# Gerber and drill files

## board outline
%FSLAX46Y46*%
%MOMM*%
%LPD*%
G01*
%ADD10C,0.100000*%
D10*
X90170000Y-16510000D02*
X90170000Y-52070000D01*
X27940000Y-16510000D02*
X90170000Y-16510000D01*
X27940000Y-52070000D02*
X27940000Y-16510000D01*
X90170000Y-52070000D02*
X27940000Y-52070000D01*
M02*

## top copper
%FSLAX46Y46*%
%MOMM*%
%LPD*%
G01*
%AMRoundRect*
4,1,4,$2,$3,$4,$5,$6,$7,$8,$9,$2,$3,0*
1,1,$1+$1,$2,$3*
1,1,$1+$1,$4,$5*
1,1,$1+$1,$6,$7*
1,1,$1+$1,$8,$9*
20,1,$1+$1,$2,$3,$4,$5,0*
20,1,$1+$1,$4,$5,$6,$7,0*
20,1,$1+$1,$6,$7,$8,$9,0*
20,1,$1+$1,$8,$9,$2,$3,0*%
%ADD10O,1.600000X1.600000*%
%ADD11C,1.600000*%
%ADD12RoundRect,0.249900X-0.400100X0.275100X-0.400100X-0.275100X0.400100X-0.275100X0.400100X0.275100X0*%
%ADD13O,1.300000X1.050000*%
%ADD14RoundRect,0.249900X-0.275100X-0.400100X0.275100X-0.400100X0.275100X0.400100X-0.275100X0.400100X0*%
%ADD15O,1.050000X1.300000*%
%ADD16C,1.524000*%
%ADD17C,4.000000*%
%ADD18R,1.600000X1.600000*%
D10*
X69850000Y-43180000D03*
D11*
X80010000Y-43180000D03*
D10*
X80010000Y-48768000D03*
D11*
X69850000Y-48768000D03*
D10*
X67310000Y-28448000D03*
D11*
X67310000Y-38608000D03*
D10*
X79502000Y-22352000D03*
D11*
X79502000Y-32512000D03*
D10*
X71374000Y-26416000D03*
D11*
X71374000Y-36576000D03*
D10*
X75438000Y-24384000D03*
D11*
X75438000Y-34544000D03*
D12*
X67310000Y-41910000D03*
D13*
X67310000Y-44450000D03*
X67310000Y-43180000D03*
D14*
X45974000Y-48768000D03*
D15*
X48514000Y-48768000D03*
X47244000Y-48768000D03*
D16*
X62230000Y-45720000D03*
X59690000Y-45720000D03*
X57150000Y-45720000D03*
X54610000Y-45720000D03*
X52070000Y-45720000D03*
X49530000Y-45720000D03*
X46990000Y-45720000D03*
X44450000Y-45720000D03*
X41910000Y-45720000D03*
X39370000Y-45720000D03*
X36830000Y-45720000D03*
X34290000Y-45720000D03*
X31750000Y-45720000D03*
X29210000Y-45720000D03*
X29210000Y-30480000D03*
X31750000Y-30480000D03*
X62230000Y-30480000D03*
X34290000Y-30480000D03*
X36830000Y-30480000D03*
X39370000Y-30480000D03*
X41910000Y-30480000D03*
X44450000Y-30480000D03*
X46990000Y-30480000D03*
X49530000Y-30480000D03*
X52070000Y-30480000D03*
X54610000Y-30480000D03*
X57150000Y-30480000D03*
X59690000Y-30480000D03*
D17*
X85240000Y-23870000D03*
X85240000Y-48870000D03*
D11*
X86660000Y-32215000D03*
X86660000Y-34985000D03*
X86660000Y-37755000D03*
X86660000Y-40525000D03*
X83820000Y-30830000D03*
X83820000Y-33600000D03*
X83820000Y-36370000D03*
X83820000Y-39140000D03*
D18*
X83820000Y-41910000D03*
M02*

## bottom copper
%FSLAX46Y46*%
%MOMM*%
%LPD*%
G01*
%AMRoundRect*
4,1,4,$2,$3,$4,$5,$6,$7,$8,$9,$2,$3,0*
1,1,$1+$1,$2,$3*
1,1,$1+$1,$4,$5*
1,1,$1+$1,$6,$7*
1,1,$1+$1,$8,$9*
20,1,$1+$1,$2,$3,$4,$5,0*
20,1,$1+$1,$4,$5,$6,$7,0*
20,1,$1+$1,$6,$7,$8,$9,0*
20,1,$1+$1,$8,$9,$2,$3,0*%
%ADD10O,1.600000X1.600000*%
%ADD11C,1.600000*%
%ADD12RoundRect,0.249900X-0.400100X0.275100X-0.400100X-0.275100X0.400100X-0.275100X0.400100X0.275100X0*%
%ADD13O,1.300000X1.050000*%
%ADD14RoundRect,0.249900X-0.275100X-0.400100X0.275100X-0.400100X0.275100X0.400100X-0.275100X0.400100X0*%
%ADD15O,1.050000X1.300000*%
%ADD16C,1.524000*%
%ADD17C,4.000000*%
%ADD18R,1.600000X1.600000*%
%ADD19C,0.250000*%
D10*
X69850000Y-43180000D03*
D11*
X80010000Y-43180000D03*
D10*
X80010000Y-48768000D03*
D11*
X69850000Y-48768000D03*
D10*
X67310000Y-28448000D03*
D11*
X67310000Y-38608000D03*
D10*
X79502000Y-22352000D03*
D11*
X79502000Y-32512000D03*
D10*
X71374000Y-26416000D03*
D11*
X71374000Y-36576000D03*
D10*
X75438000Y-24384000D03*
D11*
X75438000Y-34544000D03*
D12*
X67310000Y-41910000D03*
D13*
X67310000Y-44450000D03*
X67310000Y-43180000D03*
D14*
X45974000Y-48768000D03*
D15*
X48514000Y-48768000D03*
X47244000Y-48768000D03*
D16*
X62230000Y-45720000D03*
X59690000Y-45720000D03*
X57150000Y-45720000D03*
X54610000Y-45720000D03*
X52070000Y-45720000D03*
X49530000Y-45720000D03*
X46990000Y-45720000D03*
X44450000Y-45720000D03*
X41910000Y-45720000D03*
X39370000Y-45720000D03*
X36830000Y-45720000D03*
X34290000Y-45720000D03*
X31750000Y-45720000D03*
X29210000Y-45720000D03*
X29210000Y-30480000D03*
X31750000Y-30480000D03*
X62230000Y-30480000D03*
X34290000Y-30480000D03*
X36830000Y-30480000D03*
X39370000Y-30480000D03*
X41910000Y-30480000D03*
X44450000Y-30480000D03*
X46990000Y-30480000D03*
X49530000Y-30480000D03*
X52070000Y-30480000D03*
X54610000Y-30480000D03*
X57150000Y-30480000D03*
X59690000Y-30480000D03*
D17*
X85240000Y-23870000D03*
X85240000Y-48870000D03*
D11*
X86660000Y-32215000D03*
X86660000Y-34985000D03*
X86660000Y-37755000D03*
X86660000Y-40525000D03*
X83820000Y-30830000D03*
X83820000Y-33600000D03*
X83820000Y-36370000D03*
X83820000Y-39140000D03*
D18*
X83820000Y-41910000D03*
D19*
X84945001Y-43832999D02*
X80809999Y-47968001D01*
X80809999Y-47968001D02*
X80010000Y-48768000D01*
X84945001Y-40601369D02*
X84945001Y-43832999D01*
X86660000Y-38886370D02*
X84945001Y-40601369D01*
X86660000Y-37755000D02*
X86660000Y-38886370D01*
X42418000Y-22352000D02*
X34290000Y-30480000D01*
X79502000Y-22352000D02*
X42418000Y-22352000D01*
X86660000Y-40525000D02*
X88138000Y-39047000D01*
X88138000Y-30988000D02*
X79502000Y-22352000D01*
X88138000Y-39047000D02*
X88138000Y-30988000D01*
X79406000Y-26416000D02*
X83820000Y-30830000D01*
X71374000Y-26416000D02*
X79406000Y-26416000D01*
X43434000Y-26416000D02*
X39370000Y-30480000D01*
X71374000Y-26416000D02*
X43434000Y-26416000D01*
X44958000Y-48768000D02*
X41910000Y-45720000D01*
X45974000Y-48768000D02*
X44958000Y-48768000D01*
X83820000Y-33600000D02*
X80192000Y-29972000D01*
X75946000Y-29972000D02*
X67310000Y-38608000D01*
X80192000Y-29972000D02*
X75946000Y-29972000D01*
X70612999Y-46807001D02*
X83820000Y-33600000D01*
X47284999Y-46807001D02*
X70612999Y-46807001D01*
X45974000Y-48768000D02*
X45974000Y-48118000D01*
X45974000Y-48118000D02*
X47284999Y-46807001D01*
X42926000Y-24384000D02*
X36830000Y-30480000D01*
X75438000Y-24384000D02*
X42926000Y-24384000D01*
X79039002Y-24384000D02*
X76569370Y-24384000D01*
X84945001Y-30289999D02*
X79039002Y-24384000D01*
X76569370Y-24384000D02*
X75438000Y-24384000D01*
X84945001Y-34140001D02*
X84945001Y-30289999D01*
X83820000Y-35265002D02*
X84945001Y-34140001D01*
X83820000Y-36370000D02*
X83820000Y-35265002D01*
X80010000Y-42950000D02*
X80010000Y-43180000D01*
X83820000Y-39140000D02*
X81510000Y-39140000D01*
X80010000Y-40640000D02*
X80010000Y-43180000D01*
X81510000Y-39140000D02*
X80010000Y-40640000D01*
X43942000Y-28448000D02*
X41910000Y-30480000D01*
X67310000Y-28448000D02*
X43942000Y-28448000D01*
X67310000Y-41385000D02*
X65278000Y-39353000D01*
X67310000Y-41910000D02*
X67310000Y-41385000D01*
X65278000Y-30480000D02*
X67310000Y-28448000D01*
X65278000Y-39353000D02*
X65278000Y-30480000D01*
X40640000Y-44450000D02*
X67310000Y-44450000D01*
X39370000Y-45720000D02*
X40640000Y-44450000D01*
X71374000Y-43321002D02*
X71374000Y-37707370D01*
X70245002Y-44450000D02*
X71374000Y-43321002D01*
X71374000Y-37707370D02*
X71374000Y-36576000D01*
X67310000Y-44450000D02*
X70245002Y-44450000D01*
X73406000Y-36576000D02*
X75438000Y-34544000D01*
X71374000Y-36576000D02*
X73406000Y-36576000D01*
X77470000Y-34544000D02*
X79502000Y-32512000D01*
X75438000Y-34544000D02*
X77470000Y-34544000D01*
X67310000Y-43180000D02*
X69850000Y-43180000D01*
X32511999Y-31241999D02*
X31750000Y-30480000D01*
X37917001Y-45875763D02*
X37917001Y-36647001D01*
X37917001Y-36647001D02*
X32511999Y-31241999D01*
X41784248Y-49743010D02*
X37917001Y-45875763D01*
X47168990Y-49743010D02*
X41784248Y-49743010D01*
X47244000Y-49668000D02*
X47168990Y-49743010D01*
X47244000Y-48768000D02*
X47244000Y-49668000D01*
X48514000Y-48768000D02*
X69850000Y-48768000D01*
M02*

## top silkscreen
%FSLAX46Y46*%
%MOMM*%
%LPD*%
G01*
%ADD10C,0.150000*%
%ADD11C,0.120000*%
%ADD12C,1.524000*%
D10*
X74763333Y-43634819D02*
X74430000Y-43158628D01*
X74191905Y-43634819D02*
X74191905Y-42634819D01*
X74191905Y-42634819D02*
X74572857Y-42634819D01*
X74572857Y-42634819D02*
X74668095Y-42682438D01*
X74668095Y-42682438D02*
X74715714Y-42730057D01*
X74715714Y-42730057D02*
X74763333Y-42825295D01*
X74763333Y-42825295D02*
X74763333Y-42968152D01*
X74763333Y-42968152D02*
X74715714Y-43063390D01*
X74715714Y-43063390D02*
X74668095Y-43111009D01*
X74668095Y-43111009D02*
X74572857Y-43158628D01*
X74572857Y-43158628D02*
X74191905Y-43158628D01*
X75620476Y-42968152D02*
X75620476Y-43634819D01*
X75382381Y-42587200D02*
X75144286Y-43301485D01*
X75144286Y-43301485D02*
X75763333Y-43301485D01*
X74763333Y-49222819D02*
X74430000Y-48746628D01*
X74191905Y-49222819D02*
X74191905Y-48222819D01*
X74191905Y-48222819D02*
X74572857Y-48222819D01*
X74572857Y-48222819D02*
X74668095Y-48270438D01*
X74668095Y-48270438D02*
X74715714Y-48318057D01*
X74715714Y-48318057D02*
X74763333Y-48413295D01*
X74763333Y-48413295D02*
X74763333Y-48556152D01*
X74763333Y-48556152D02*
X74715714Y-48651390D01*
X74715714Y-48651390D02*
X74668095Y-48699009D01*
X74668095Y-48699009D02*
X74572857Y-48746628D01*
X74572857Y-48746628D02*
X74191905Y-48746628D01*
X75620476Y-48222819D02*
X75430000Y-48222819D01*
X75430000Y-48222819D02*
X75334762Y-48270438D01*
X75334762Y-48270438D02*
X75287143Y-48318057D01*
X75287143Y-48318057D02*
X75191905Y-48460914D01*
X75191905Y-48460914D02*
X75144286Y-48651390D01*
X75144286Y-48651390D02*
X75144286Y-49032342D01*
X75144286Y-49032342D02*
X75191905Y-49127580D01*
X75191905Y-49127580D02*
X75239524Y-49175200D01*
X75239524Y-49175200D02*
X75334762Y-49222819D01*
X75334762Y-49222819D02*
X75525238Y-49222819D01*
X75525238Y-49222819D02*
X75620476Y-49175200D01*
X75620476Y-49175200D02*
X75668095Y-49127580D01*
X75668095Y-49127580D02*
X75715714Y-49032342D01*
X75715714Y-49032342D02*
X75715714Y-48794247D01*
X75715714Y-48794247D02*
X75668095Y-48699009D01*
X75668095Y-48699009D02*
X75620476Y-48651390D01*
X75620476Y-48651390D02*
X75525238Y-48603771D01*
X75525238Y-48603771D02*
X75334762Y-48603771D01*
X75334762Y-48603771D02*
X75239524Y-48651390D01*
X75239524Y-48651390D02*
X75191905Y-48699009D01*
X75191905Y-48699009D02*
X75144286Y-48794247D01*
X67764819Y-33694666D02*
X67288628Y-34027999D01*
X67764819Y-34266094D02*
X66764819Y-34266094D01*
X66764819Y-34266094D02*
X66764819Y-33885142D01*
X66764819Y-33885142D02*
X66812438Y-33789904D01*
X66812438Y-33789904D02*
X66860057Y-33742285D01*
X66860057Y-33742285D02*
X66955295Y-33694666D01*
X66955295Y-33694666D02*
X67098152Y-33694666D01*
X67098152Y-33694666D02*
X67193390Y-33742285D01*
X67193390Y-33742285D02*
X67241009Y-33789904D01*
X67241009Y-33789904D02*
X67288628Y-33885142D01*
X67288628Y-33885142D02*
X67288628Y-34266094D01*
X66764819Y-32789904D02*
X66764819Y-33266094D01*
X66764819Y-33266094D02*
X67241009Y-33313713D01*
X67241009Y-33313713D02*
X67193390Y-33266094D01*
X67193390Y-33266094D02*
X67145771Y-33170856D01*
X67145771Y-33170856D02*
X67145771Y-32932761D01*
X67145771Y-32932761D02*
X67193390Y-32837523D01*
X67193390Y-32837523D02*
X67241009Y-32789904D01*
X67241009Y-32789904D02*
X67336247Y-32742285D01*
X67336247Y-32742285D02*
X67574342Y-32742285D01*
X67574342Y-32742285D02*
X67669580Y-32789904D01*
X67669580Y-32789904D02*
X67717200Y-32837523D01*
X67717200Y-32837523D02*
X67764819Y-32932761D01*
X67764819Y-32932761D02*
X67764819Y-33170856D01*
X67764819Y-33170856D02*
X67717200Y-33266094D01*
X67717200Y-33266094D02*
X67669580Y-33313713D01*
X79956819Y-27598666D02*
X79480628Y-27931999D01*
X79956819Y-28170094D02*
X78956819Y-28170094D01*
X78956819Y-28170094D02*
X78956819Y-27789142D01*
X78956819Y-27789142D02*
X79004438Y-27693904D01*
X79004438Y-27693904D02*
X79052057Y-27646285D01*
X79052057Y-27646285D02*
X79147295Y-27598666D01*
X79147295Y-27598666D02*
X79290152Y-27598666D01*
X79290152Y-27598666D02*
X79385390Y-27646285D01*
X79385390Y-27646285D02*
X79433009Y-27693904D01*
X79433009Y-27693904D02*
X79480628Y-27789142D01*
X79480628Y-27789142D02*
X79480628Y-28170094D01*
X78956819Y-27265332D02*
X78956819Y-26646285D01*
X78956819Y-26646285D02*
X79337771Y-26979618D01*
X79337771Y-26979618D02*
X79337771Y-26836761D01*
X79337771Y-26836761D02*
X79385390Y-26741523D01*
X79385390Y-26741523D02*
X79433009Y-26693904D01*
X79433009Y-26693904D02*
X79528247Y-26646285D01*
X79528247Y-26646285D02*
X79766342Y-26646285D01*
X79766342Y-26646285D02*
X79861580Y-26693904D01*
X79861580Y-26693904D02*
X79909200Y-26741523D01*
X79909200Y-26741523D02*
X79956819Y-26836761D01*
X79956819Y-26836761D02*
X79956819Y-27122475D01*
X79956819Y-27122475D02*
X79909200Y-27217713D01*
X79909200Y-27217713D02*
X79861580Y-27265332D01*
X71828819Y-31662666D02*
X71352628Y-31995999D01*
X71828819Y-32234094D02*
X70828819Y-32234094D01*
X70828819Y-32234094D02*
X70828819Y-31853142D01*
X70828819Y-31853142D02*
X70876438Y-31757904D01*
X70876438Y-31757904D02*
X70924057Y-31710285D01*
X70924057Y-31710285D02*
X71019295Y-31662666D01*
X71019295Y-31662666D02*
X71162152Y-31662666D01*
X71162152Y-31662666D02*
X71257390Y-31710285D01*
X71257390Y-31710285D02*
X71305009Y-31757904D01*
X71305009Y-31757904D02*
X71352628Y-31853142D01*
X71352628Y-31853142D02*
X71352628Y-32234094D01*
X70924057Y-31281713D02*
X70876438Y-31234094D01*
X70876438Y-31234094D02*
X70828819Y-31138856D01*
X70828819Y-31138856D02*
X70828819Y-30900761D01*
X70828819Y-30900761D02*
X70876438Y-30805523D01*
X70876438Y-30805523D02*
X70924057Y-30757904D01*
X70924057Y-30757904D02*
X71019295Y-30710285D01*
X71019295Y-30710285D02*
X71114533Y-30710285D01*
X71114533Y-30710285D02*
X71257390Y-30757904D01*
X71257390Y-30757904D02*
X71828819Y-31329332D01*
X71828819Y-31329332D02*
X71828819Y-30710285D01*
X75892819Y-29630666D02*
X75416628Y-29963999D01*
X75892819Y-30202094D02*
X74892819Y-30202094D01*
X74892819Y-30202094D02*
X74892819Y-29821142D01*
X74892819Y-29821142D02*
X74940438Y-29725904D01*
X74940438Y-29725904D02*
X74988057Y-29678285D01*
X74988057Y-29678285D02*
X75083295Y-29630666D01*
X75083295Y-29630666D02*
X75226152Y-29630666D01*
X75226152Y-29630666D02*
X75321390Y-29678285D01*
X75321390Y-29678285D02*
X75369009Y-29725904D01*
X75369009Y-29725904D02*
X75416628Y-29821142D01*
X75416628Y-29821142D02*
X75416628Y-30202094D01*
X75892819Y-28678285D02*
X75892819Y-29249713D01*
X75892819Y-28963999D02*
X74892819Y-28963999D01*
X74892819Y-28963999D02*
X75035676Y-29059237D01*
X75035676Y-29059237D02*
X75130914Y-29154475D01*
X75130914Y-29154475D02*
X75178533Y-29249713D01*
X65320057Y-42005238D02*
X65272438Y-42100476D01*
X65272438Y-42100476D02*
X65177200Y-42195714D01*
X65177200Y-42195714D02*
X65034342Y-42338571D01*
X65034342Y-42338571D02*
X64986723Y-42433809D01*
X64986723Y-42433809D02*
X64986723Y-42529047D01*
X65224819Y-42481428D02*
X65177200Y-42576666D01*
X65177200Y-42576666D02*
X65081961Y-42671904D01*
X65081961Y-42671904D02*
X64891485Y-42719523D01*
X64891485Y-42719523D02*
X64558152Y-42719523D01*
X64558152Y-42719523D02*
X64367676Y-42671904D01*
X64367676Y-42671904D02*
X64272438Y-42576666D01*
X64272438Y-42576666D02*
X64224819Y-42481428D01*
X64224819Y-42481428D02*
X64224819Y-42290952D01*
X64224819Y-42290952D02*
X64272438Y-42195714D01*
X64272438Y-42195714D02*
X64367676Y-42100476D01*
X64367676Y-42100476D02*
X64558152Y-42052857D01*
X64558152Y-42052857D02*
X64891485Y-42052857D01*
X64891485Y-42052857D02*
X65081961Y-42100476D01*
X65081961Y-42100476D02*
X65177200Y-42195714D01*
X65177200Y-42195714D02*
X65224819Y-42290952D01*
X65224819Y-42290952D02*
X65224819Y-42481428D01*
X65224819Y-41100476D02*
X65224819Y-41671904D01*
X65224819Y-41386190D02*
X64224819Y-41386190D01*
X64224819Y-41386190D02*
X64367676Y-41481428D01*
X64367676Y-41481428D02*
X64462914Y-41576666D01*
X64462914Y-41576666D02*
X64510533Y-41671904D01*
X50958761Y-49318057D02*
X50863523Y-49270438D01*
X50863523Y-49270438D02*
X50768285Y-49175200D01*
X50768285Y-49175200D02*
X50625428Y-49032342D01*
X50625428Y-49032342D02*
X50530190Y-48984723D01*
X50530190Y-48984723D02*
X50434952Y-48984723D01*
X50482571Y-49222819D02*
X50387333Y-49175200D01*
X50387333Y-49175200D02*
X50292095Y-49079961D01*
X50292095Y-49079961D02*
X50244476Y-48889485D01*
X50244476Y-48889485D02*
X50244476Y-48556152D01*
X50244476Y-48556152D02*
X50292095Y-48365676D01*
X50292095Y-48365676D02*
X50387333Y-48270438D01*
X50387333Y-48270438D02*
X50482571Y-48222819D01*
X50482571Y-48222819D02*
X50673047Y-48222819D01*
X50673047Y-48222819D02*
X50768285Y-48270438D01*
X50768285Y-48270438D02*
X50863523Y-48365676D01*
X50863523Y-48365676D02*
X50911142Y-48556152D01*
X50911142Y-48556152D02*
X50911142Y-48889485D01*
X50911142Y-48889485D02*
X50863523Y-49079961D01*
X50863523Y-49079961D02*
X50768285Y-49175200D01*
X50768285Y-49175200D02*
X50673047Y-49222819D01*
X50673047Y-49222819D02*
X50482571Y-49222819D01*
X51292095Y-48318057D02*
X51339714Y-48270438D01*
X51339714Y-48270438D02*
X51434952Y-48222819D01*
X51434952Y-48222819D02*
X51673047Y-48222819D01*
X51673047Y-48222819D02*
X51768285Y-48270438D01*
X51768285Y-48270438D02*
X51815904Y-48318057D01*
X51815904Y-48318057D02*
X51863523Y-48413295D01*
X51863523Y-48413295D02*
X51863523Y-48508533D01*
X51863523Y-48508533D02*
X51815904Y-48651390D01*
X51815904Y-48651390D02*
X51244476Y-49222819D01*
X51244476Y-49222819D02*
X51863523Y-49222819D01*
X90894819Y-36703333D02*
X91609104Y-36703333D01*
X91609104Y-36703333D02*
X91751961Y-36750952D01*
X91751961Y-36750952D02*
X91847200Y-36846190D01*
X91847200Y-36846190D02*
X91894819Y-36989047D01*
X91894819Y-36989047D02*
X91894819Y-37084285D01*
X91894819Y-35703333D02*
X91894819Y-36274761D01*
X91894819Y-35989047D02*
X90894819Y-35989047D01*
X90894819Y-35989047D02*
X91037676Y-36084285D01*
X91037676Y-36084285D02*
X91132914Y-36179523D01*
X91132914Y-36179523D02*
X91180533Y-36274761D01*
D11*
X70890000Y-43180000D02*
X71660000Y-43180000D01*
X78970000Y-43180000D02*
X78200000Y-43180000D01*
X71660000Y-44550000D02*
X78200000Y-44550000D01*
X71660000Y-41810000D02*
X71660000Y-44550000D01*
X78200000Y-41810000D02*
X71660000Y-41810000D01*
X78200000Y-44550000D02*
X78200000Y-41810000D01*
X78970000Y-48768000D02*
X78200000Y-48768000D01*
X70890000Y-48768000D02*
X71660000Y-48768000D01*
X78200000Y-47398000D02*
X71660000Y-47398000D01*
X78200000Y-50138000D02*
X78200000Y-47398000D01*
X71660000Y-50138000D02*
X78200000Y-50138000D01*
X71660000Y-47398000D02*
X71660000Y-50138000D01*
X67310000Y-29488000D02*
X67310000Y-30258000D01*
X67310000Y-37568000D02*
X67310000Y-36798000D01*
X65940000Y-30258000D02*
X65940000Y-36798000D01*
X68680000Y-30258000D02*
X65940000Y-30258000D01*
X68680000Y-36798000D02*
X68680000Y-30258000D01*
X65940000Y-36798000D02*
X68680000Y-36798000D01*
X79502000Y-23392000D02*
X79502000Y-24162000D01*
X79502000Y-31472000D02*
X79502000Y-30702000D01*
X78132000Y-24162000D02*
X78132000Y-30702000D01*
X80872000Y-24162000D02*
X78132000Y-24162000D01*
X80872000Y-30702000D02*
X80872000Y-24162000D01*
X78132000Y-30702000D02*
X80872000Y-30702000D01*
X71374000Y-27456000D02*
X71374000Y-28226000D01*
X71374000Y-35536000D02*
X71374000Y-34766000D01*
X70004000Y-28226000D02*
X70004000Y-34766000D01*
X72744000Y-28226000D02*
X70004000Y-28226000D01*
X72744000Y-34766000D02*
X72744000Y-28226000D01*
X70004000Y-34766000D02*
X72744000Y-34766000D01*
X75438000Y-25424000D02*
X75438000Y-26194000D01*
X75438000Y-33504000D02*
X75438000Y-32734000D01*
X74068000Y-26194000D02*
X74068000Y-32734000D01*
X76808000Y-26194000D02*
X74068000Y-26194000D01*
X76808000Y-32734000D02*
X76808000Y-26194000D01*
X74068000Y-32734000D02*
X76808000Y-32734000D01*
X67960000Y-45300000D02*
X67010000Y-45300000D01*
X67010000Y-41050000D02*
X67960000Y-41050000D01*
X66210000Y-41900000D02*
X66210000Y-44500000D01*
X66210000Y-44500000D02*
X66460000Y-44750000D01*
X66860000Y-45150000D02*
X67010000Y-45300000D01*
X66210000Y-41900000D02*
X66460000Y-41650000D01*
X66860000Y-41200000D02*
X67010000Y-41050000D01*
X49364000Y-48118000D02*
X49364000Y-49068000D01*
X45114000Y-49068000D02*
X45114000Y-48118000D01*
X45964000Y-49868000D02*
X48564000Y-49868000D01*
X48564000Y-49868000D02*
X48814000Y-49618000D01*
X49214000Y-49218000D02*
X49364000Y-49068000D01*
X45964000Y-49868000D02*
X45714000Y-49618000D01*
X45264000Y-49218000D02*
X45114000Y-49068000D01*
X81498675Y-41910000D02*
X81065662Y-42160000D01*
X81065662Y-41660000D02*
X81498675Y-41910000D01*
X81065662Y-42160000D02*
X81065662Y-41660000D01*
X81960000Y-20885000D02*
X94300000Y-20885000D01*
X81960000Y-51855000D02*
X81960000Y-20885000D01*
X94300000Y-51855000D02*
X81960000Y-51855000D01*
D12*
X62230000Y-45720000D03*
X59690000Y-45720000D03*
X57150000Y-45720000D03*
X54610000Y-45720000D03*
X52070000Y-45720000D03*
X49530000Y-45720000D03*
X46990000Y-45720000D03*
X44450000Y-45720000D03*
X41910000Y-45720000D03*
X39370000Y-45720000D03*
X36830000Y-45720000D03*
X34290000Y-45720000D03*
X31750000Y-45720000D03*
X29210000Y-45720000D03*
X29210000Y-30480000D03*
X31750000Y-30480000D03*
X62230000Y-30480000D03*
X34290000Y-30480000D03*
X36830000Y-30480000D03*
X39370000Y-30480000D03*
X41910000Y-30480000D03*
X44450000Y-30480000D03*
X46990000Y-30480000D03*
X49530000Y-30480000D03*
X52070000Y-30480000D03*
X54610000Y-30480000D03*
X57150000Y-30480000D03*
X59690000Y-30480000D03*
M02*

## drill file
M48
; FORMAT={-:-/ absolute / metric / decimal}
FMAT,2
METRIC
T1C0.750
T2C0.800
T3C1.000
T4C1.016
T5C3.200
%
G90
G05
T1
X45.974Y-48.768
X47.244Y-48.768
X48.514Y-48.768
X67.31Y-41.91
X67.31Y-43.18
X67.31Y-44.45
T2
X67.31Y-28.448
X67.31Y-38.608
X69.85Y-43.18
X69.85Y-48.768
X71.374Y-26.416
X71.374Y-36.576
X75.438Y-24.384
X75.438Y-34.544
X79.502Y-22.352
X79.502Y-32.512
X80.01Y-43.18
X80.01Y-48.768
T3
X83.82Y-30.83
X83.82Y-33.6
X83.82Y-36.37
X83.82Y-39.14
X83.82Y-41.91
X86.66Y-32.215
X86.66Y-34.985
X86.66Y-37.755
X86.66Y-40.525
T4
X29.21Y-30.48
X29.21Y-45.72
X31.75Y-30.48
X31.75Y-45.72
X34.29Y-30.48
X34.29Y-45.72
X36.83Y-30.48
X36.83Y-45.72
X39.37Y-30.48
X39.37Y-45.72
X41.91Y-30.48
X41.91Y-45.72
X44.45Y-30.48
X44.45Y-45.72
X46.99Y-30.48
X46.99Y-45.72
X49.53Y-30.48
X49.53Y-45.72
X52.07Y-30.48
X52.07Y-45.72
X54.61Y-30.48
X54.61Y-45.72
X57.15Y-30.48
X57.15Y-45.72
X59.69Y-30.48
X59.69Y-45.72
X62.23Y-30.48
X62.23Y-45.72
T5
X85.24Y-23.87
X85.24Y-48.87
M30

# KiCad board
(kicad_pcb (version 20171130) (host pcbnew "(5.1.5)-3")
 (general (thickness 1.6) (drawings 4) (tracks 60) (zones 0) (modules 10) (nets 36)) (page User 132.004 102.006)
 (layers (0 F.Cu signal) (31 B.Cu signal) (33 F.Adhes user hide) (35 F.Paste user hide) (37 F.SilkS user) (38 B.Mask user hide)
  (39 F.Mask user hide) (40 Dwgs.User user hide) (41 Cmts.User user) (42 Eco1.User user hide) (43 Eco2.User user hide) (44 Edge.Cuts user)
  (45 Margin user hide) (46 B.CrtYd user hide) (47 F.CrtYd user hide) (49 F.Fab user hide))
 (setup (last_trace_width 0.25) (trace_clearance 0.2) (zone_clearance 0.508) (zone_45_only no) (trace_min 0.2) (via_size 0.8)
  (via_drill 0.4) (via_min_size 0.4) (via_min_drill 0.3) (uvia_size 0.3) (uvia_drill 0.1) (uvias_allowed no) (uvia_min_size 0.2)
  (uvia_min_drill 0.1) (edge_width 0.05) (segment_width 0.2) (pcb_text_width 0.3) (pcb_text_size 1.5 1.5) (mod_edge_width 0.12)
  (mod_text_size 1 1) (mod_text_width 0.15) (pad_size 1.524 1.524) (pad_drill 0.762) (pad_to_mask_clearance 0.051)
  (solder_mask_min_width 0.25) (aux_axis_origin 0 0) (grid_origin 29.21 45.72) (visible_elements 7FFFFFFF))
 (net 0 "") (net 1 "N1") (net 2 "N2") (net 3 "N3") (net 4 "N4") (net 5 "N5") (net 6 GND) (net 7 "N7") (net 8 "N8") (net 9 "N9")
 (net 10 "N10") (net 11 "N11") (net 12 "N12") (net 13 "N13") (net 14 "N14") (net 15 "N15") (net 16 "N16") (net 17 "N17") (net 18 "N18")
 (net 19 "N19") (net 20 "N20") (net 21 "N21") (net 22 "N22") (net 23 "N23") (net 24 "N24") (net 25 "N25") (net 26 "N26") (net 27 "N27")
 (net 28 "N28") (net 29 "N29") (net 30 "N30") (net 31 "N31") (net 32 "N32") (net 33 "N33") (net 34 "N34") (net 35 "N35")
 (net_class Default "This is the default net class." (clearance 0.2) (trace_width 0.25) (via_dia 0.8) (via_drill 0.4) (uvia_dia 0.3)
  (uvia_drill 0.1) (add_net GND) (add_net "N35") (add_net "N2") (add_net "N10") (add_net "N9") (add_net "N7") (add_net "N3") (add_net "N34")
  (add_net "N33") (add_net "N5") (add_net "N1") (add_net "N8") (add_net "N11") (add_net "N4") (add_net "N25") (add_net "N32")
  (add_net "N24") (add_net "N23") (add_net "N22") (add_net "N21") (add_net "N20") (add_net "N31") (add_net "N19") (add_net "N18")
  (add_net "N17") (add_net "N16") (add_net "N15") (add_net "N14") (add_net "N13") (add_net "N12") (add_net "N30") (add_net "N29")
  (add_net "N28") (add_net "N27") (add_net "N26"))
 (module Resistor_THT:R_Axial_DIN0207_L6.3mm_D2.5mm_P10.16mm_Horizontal (layer F.Cu) (at 80.01 43.18 180)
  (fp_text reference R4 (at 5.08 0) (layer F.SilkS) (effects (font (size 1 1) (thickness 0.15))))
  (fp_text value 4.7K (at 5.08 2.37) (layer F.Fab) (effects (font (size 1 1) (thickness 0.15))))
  (fp_line (start 9.12 0) (end 8.35 0) (layer F.SilkS) (width 0.12))
  (fp_line (start 1.04 0) (end 1.81 0) (layer F.SilkS) (width 0.12))
  (fp_line (start 8.35 -1.37) (end 1.81 -1.37) (layer F.SilkS) (width 0.12))
  (fp_line (start 8.35 1.37) (end 8.35 -1.37) (layer F.SilkS) (width 0.12))
  (fp_line (start 1.81 1.37) (end 8.35 1.37) (layer F.SilkS) (width 0.12))
  (fp_line (start 1.81 -1.37) (end 1.81 1.37) (layer F.SilkS) (width 0.12))
  (pad 2 thru_hole oval (at 10.16 0 180) (size 1.6 1.6) (drill 0.8) (layers *.Cu *.Mask) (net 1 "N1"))
  (pad 1 thru_hole circle (at 0 0 180) (size 1.6 1.6) (drill 0.8) (layers *.Cu *.Mask) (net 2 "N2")))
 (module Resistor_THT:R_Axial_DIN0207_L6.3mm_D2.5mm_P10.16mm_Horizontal (layer F.Cu) (at 69.85 48.768)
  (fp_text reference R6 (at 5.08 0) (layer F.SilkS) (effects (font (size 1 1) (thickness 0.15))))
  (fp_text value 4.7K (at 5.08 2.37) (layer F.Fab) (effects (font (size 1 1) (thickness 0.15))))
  (fp_line (start 9.12 0) (end 8.35 0) (layer F.SilkS) (width 0.12))
  (fp_line (start 1.04 0) (end 1.81 0) (layer F.SilkS) (width 0.12))
  (fp_line (start 8.35 -1.37) (end 1.81 -1.37) (layer F.SilkS) (width 0.12))
  (fp_line (start 8.35 1.37) (end 8.35 -1.37) (layer F.SilkS) (width 0.12))
  (fp_line (start 1.81 1.37) (end 8.35 1.37) (layer F.SilkS) (width 0.12))
  (fp_line (start 1.81 -1.37) (end 1.81 1.37) (layer F.SilkS) (width 0.12))
  (pad 2 thru_hole oval (at 10.16 0) (size 1.6 1.6) (drill 0.8) (layers *.Cu *.Mask) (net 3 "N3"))
  (pad 1 thru_hole circle (at 0 0) (size 1.6 1.6) (drill 0.8) (layers *.Cu *.Mask) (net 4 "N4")))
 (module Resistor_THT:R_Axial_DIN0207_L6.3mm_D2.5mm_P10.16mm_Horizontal (layer F.Cu) (at 67.31 38.608 90)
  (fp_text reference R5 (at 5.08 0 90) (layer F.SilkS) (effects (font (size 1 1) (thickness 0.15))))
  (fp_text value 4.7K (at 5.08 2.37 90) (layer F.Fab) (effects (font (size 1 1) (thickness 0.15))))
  (fp_line (start 9.12 0) (end 8.35 0) (layer F.SilkS) (width 0.12))
  (fp_line (start 1.04 0) (end 1.81 0) (layer F.SilkS) (width 0.12))
  (fp_line (start 8.35 -1.37) (end 1.81 -1.37) (layer F.SilkS) (width 0.12))
  (fp_line (start 8.35 1.37) (end 8.35 -1.37) (layer F.SilkS) (width 0.12))
  (fp_line (start 1.81 1.37) (end 8.35 1.37) (layer F.SilkS) (width 0.12))
  (fp_line (start 1.81 -1.37) (end 1.81 1.37) (layer F.SilkS) (width 0.12))
  (pad 2 thru_hole oval (at 10.16 0 90) (size 1.6 1.6) (drill 0.8) (layers *.Cu *.Mask) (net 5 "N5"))
  (pad 1 thru_hole circle (at 0 0 90) (size 1.6 1.6) (drill 0.8) (layers *.Cu *.Mask) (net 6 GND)))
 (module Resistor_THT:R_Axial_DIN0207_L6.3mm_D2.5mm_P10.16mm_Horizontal (layer F.Cu) (at 79.502 32.512 90)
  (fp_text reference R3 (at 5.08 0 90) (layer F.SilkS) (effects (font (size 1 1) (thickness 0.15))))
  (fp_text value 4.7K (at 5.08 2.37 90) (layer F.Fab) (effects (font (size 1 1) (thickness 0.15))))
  (fp_line (start 9.12 0) (end 8.35 0) (layer F.SilkS) (width 0.12))
  (fp_line (start 1.04 0) (end 1.81 0) (layer F.SilkS) (width 0.12))
  (fp_line (start 8.35 -1.37) (end 1.81 -1.37) (layer F.SilkS) (width 0.12))
  (fp_line (start 8.35 1.37) (end 8.35 -1.37) (layer F.SilkS) (width 0.12))
  (fp_line (start 1.81 1.37) (end 8.35 1.37) (layer F.SilkS) (width 0.12))
  (fp_line (start 1.81 -1.37) (end 1.81 1.37) (layer F.SilkS) (width 0.12))
  (pad 2 thru_hole oval (at 10.16 0 90) (size 1.6 1.6) (drill 0.8) (layers *.Cu *.Mask) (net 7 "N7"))
  (pad 1 thru_hole circle (at 0 0 90) (size 1.6 1.6) (drill 0.8) (layers *.Cu *.Mask) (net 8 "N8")))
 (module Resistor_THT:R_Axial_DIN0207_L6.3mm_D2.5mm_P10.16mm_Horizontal (layer F.Cu) (at 71.374 36.576 90)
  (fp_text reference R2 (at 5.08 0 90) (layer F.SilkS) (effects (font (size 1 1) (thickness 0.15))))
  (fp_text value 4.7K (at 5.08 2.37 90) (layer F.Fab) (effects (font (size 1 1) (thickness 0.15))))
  (fp_line (start 9.12 0) (end 8.35 0) (layer F.SilkS) (width 0.12))
  (fp_line (start 1.04 0) (end 1.81 0) (layer F.SilkS) (width 0.12))
  (fp_line (start 8.35 -1.37) (end 1.81 -1.37) (layer F.SilkS) (width 0.12))
  (fp_line (start 8.35 1.37) (end 8.35 -1.37) (layer F.SilkS) (width 0.12))
  (fp_line (start 1.81 1.37) (end 8.35 1.37) (layer F.SilkS) (width 0.12))
  (fp_line (start 1.81 -1.37) (end 1.81 1.37) (layer F.SilkS) (width 0.12))
  (pad 2 thru_hole oval (at 10.16 0 90) (size 1.6 1.6) (drill 0.8) (layers *.Cu *.Mask) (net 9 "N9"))
  (pad 1 thru_hole circle (at 0 0 90) (size 1.6 1.6) (drill 0.8) (layers *.Cu *.Mask) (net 8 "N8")))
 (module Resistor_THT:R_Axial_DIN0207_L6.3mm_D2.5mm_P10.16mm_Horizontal (layer F.Cu) (at 75.438 34.544 90)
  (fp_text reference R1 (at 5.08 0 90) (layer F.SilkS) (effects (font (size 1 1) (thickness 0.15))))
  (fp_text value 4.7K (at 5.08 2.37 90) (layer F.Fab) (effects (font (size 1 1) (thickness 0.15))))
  (fp_line (start 9.12 0) (end 8.35 0) (layer F.SilkS) (width 0.12))
  (fp_line (start 1.04 0) (end 1.81 0) (layer F.SilkS) (width 0.12))
  (fp_line (start 8.35 -1.37) (end 1.81 -1.37) (layer F.SilkS) (width 0.12))
  (fp_line (start 8.35 1.37) (end 8.35 -1.37) (layer F.SilkS) (width 0.12))
  (fp_line (start 1.81 1.37) (end 8.35 1.37) (layer F.SilkS) (width 0.12))
  (fp_line (start 1.81 -1.37) (end 1.81 1.37) (layer F.SilkS) (width 0.12))
  (pad 2 thru_hole oval (at 10.16 0 90) (size 1.6 1.6) (drill 0.8) (layers *.Cu *.Mask) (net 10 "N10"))
  (pad 1 thru_hole circle (at 0 0 90) (size 1.6 1.6) (drill 0.8) (layers *.Cu *.Mask) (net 8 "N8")))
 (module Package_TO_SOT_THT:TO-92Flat (layer F.Cu) (at 67.31 41.91 270)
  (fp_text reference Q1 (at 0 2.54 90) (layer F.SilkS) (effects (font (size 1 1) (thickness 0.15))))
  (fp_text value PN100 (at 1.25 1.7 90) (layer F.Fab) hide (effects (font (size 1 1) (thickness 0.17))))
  (fp_line (start 3.39 -0.65) (end 3.39 0.3) (layer F.SilkS) (width 0.12))
  (fp_line (start -0.86 0.3) (end -0.86 -0.65) (layer F.SilkS) (width 0.12))
  (fp_line (start -0.01 1.1) (end 2.59 1.1) (layer F.SilkS) (width 0.12))
  (fp_line (start 2.59 1.1) (end 2.84 0.85) (layer F.SilkS) (width 0.12))
  (fp_line (start 3.24 0.45) (end 3.39 0.3) (layer F.SilkS) (width 0.12))
  (fp_line (start -0.01 1.1) (end -0.26 0.85) (layer F.SilkS) (width 0.12))
  (fp_line (start -0.71 0.45) (end -0.86 0.3) (layer F.SilkS) (width 0.12))
  (pad 1 thru_hole roundrect (at 0 0 270) (size 1.05 1.3) (drill 0.75) (layers *.Cu *.Mask) (roundrect_rratio 0.238) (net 5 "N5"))
  (pad 3 thru_hole oval (at 2.54 0 270) (size 1.05 1.3) (drill 0.75) (layers *.Cu *.Mask) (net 8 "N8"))
  (pad 2 thru_hole oval (at 1.27 0 270) (size 1.05 1.3) (drill 0.75) (layers *.Cu *.Mask) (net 1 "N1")))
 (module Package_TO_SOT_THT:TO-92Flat (layer F.Cu) (at 45.974 48.768)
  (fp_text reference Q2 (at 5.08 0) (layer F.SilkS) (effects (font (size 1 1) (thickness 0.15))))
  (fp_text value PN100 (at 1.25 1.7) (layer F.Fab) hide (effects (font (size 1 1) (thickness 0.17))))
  (fp_line (start 3.39 -0.65) (end 3.39 0.3) (layer F.SilkS) (width 0.12))
  (fp_line (start -0.86 0.3) (end -0.86 -0.65) (layer F.SilkS) (width 0.12))
  (fp_line (start -0.01 1.1) (end 2.59 1.1) (layer F.SilkS) (width 0.12))
  (fp_line (start 2.59 1.1) (end 2.84 0.85) (layer F.SilkS) (width 0.12))
  (fp_line (start 3.24 0.45) (end 3.39 0.3) (layer F.SilkS) (width 0.12))
  (fp_line (start -0.01 1.1) (end -0.26 0.85) (layer F.SilkS) (width 0.12))
  (fp_line (start -0.71 0.45) (end -0.86 0.3) (layer F.SilkS) (width 0.12))
  (pad 1 thru_hole roundrect (at 0 0) (size 1.05 1.3) (drill 0.75) (layers *.Cu *.Mask) (roundrect_rratio 0.238) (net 6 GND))
  (pad 3 thru_hole oval (at 2.54 0) (size 1.05 1.3) (drill 0.75) (layers *.Cu *.Mask) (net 4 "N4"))
  (pad 2 thru_hole oval (at 1.27 0) (size 1.05 1.3) (drill 0.75) (layers *.Cu *.Mask) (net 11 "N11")))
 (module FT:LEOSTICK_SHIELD (layer F.Cu) (at 29.21 45.72)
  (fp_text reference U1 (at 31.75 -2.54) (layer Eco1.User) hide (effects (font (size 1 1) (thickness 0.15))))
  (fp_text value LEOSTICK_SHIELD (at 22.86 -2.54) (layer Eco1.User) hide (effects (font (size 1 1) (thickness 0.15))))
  (pad 27 thru_hole circle (at 33.02 0 180) (size 1.524 1.524) (drill 1.016) (layers *.Cu *.Mask F.SilkS) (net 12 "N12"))
  (pad 26 thru_hole circle (at 30.48 0 180) (size 1.524 1.524) (drill 1.016) (layers *.Cu *.Mask F.SilkS) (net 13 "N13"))
  (pad 25 thru_hole circle (at 27.94 0 180) (size 1.524 1.524) (drill 1.016) (layers *.Cu *.Mask F.SilkS) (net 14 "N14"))
  (pad 24 thru_hole circle (at 25.4 0 180) (size 1.524 1.524) (drill 1.016) (layers *.Cu *.Mask F.SilkS) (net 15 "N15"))
  (pad 23 thru_hole circle (at 22.86 0 180) (size 1.524 1.524) (drill 1.016) (layers *.Cu *.Mask F.SilkS) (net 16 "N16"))
  (pad 22 thru_hole circle (at 20.32 0 180) (size 1.524 1.524) (drill 1.016) (layers *.Cu *.Mask F.SilkS) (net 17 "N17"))
  (pad 21 thru_hole circle (at 17.78 0 180) (size 1.524 1.524) (drill 1.016) (layers *.Cu *.Mask F.SilkS) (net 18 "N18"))
  (pad 20 thru_hole circle (at 15.24 0 180) (size 1.524 1.524) (drill 1.016) (layers *.Cu *.Mask F.SilkS) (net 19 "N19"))
  (pad 19 thru_hole circle (at 12.7 0 180) (size 1.524 1.524) (drill 1.016) (layers *.Cu *.Mask F.SilkS) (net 6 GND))
  (pad 18 thru_hole circle (at 10.16 0 180) (size 1.524 1.524) (drill 1.016) (layers *.Cu *.Mask F.SilkS) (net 8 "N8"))
  (pad 17 thru_hole circle (at 7.62 0 180) (size 1.524 1.524) (drill 1.016) (layers *.Cu *.Mask F.SilkS) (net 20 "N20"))
  (pad 16 thru_hole circle (at 5.08 0 180) (size 1.524 1.524) (drill 1.016) (layers *.Cu *.Mask F.SilkS) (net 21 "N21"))
  (pad 15 thru_hole circle (at 2.54 0 180) (size 1.524 1.524) (drill 1.016) (layers *.Cu *.Mask F.SilkS) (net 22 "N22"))
  (pad 14 thru_hole circle (at 0 0 180) (size 1.524 1.524) (drill 1.016) (layers *.Cu *.Mask F.SilkS) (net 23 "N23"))
  (pad 13 thru_hole circle (at 0 -15.24 180) (size 1.524 1.524) (drill 1.016) (layers *.Cu *.Mask F.SilkS) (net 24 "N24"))
  (pad 12 thru_hole circle (at 2.54 -15.24 180) (size 1.524 1.524) (drill 1.016) (layers *.Cu *.Mask F.SilkS) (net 11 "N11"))
  (pad 0 thru_hole circle (at 33.02 -15.24 180) (size 1.524 1.524) (drill 1.016) (layers *.Cu *.Mask F.SilkS) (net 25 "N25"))
  (pad 11 thru_hole circle (at 5.08 -15.24 180) (size 1.524 1.524) (drill 1.016) (layers *.Cu *.Mask F.SilkS) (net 7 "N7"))
  (pad 10 thru_hole circle (at 7.62 -15.24 180) (size 1.524 1.524) (drill 1.016) (layers *.Cu *.Mask F.SilkS) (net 10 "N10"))
  (pad 9 thru_hole circle (at 10.16 -15.24 180) (size 1.524 1.524) (drill 1.016) (layers *.Cu *.Mask F.SilkS) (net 9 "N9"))
  (pad 8 thru_hole circle (at 12.7 -15.24 180) (size 1.524 1.524) (drill 1.016) (layers *.Cu *.Mask F.SilkS) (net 5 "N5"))
  (pad 7 thru_hole circle (at 15.24 -15.24 180) (size 1.524 1.524) (drill 1.016) (layers *.Cu *.Mask F.SilkS) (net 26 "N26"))
  (pad 6 thru_hole circle (at 17.78 -15.24 180) (size 1.524 1.524) (drill 1.016) (layers *.Cu *.Mask F.SilkS) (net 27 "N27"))
  (pad 5 thru_hole circle (at 20.32 -15.24 180) (size 1.524 1.524) (drill 1.016) (layers *.Cu *.Mask F.SilkS) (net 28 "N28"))
  (pad 4 thru_hole circle (at 22.86 -15.24 180) (size 1.524 1.524) (drill 1.016) (layers *.Cu *.Mask F.SilkS) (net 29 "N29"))
  (pad 3 thru_hole circle (at 25.4 -15.24 180) (size 1.524 1.524) (drill 1.016) (layers *.Cu *.Mask F.SilkS) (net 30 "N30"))
  (pad 2 thru_hole circle (at 27.94 -15.24 180) (size 1.524 1.524) (drill 1.016) (layers *.Cu *.Mask F.SilkS) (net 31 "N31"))
  (pad 1 thru_hole circle (at 30.48 -15.24 180) (size 1.524 1.524) (drill 1.016) (layers *.Cu *.Mask F.SilkS) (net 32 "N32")))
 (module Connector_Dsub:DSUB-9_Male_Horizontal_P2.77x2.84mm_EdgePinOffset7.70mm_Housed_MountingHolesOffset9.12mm (layer F.Cu)
  (at 83.82 41.91 90)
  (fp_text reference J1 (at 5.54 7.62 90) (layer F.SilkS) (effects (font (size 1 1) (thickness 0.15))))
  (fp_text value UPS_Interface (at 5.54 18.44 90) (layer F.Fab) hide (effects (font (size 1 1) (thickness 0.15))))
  (fp_line (start 0 -2.321325) (end -0.25 -2.754338) (layer F.SilkS) (width 0.12))
  (fp_line (start 0.25 -2.754338) (end 0 -2.321325) (layer F.SilkS) (width 0.12))
  (fp_line (start -0.25 -2.754338) (end 0.25 -2.754338) (layer F.SilkS) (width 0.12))
  (fp_line (start 21.025 -1.86) (end 21.025 10.48) (layer F.SilkS) (width 0.12))
  (fp_line (start -9.945 -1.86) (end 21.025 -1.86) (layer F.SilkS) (width 0.12))
  (fp_line (start -9.945 10.48) (end -9.945 -1.86) (layer F.SilkS) (width 0.12))
  (pad 0 thru_hole circle (at 18.04 1.42 90) (size 4 4) (drill 3.2) (layers *.Cu *.Mask))
  (pad 0 thru_hole circle (at -6.96 1.42 90) (size 4 4) (drill 3.2) (layers *.Cu *.Mask))
  (pad 9 thru_hole circle (at 9.695 2.84 90) (size 1.6 1.6) (drill 1) (layers *.Cu *.Mask) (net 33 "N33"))
  (pad 8 thru_hole circle (at 6.925 2.84 90) (size 1.6 1.6) (drill 1) (layers *.Cu *.Mask) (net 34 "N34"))
  (pad 7 thru_hole circle (at 4.155 2.84 90) (size 1.6 1.6) (drill 1) (layers *.Cu *.Mask) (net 3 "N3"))
  (pad 6 thru_hole circle (at 1.385 2.84 90) (size 1.6 1.6) (drill 1) (layers *.Cu *.Mask) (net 7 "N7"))
  (pad 5 thru_hole circle (at 11.08 0 90) (size 1.6 1.6) (drill 1) (layers *.Cu *.Mask) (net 9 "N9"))
  (pad 4 thru_hole circle (at 8.31 0 90) (size 1.6 1.6) (drill 1) (layers *.Cu *.Mask) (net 6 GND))
  (pad 3 thru_hole circle (at 5.54 0 90) (size 1.6 1.6) (drill 1) (layers *.Cu *.Mask) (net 10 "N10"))
  (pad 2 thru_hole circle (at 2.77 0 90) (size 1.6 1.6) (drill 1) (layers *.Cu *.Mask) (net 2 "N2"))
  (pad 1 thru_hole rect (at 0 0 90) (size 1.6 1.6) (drill 1) (layers *.Cu *.Mask) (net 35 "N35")))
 (gr_line (start 90.17 16.51) (end 90.17 52.07) (layer Edge.Cuts) (width 0.1))
 (gr_line (start 27.94 16.51) (end 90.17 16.51) (layer Edge.Cuts) (width 0.1))
 (gr_line (start 27.94 52.07) (end 27.94 16.51) (layer Edge.Cuts) (width 0.1))
 (gr_line (start 90.17 52.07) (end 27.94 52.07) (layer Edge.Cuts) (width 0.1))
 (segment (start 84.945001 43.832999) (end 80.809999 47.968001) (width 0.25) (layer B.Cu) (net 3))
 (segment (start 80.809999 47.968001) (end 80.01 48.768) (width 0.25) (layer B.Cu) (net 3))
 (segment (start 84.945001 40.601369) (end 84.945001 43.832999) (width 0.25) (layer B.Cu) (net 3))
 (segment (start 86.66 38.88637) (end 84.945001 40.601369) (width 0.25) (layer B.Cu) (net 3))
 (segment (start 86.66 37.755) (end 86.66 38.88637) (width 0.25) (layer B.Cu) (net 3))
 (segment (start 42.418 22.352) (end 34.29 30.48) (width 0.25) (layer B.Cu) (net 7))
 (segment (start 79.502 22.352) (end 42.418 22.352) (width 0.25) (layer B.Cu) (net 7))
 (segment (start 86.66 40.525) (end 88.138 39.047) (width 0.25) (layer B.Cu) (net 7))
 (segment (start 88.138 30.988) (end 79.502 22.352) (width 0.25) (layer B.Cu) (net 7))
 (segment (start 88.138 39.047) (end 88.138 30.988) (width 0.25) (layer B.Cu) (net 7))
 (segment (start 79.406 26.416) (end 83.82 30.83) (width 0.25) (layer B.Cu) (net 9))
 (segment (start 71.374 26.416) (end 79.406 26.416) (width 0.25) (layer B.Cu) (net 9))
 (segment (start 43.434 26.416) (end 39.37 30.48) (width 0.25) (layer B.Cu) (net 9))
 (segment (start 71.374 26.416) (end 43.434 26.416) (width 0.25) (layer B.Cu) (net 9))
 (segment (start 44.958 48.768) (end 41.91 45.72) (width 0.25) (layer B.Cu) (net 6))
 (segment (start 45.974 48.768) (end 44.958 48.768) (width 0.25) (layer B.Cu) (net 6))
 (segment (start 83.82 33.6) (end 80.192 29.972) (width 0.25) (layer B.Cu) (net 6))
 (segment (start 75.946 29.972) (end 67.31 38.608) (width 0.25) (layer B.Cu) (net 6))
 (segment (start 80.192 29.972) (end 75.946 29.972) (width 0.25) (layer B.Cu) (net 6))
 (segment (start 70.612999 46.807001) (end 83.82 33.6) (width 0.25) (layer B.Cu) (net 6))
 (segment (start 47.284999 46.807001) (end 70.612999 46.807001) (width 0.25) (layer B.Cu) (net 6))
 (segment (start 45.974 48.768) (end 45.974 48.118) (width 0.25) (layer B.Cu) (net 6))
 (segment (start 45.974 48.118) (end 47.284999 46.807001) (width 0.25) (layer B.Cu) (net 6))
 (segment (start 42.926 24.384) (end 36.83 30.48) (width 0.25) (layer B.Cu) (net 10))
 (segment (start 75.438 24.384) (end 42.926 24.384) (width 0.25) (layer B.Cu) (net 10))
 (segment (start 79.039002 24.384) (end 76.56937 24.384) (width 0.25) (layer B.Cu) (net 10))
 (segment (start 84.945001 30.289999) (end 79.039002 24.384) (width 0.25) (layer B.Cu) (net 10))
 (segment (start 76.56937 24.384) (end 75.438 24.384) (width 0.25) (layer B.Cu) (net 10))
 (segment (start 84.945001 34.140001) (end 84.945001 30.289999) (width 0.25) (layer B.Cu) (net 10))
 (segment (start 83.82 35.265002) (end 84.945001 34.140001) (width 0.25) (layer B.Cu) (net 10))
 (segment (start 83.82 36.37) (end 83.82 35.265002) (width 0.25) (layer B.Cu) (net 10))
 (segment (start 80.01 42.95) (end 80.01 43.18) (width 0.25) (layer B.Cu) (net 2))
 (segment (start 83.82 39.14) (end 81.51 39.14) (width 0.25) (layer B.Cu) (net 2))
 (segment (start 80.01 40.64) (end 80.01 43.18) (width 0.25) (layer B.Cu) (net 2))
 (segment (start 81.51 39.14) (end 80.01 40.64) (width 0.25) (layer B.Cu) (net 2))
 (segment (start 43.942 28.448) (end 41.91 30.48) (width 0.25) (layer B.Cu) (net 5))
 (segment (start 67.31 28.448) (end 43.942 28.448) (width 0.25) (layer B.Cu) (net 5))
 (segment (start 67.31 41.385) (end 65.278 39.353) (width 0.25) (layer B.Cu) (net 5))
 (segment (start 67.31 41.91) (end 67.31 41.385) (width 0.25) (layer B.Cu) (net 5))
 (segment (start 65.278 30.48) (end 67.31 28.448) (width 0.25) (layer B.Cu) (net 5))
 (segment (start 65.278 39.353) (end 65.278 30.48) (width 0.25) (layer B.Cu) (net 5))
 (segment (start 40.64 44.45) (end 67.31 44.45) (width 0.25) (layer B.Cu) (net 8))
 (segment (start 39.37 45.72) (end 40.64 44.45) (width 0.25) (layer B.Cu) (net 8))
 (segment (start 71.374 43.321002) (end 71.374 37.70737) (width 0.25) (layer B.Cu) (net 8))
 (segment (start 70.245002 44.45) (end 71.374 43.321002) (width 0.25) (layer B.Cu) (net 8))
 (segment (start 71.374 37.70737) (end 71.374 36.576) (width 0.25) (layer B.Cu) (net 8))
 (segment (start 67.31 44.45) (end 70.245002 44.45) (width 0.25) (layer B.Cu) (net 8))
 (segment (start 73.406 36.576) (end 75.438 34.544) (width 0.25) (layer B.Cu) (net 8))
 (segment (start 71.374 36.576) (end 73.406 36.576) (width 0.25) (layer B.Cu) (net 8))
 (segment (start 77.47 34.544) (end 79.502 32.512) (width 0.25) (layer B.Cu) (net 8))
 (segment (start 75.438 34.544) (end 77.47 34.544) (width 0.25) (layer B.Cu) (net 8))
 (segment (start 67.31 43.18) (end 69.85 43.18) (width 0.25) (layer B.Cu) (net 1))
 (segment (start 32.511999 31.241999) (end 31.75 30.48) (width 0.25) (layer B.Cu) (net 11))
 (segment (start 37.917001 45.875763) (end 37.917001 36.647001) (width 0.25) (layer B.Cu) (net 11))
 (segment (start 37.917001 36.647001) (end 32.511999 31.241999) (width 0.25) (layer B.Cu) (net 11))
 (segment (start 41.784248 49.74301) (end 37.917001 45.875763) (width 0.25) (layer B.Cu) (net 11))
 (segment (start 47.16899 49.74301) (end 41.784248 49.74301) (width 0.25) (layer B.Cu) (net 11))
 (segment (start 47.244 49.668) (end 47.16899 49.74301) (width 0.25) (layer B.Cu) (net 11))
 (segment (start 47.244 48.768) (end 47.244 49.668) (width 0.25) (layer B.Cu) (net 11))
 (segment (start 48.514 48.768) (end 69.85 48.768) (width 0.25) (layer B.Cu) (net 4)))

